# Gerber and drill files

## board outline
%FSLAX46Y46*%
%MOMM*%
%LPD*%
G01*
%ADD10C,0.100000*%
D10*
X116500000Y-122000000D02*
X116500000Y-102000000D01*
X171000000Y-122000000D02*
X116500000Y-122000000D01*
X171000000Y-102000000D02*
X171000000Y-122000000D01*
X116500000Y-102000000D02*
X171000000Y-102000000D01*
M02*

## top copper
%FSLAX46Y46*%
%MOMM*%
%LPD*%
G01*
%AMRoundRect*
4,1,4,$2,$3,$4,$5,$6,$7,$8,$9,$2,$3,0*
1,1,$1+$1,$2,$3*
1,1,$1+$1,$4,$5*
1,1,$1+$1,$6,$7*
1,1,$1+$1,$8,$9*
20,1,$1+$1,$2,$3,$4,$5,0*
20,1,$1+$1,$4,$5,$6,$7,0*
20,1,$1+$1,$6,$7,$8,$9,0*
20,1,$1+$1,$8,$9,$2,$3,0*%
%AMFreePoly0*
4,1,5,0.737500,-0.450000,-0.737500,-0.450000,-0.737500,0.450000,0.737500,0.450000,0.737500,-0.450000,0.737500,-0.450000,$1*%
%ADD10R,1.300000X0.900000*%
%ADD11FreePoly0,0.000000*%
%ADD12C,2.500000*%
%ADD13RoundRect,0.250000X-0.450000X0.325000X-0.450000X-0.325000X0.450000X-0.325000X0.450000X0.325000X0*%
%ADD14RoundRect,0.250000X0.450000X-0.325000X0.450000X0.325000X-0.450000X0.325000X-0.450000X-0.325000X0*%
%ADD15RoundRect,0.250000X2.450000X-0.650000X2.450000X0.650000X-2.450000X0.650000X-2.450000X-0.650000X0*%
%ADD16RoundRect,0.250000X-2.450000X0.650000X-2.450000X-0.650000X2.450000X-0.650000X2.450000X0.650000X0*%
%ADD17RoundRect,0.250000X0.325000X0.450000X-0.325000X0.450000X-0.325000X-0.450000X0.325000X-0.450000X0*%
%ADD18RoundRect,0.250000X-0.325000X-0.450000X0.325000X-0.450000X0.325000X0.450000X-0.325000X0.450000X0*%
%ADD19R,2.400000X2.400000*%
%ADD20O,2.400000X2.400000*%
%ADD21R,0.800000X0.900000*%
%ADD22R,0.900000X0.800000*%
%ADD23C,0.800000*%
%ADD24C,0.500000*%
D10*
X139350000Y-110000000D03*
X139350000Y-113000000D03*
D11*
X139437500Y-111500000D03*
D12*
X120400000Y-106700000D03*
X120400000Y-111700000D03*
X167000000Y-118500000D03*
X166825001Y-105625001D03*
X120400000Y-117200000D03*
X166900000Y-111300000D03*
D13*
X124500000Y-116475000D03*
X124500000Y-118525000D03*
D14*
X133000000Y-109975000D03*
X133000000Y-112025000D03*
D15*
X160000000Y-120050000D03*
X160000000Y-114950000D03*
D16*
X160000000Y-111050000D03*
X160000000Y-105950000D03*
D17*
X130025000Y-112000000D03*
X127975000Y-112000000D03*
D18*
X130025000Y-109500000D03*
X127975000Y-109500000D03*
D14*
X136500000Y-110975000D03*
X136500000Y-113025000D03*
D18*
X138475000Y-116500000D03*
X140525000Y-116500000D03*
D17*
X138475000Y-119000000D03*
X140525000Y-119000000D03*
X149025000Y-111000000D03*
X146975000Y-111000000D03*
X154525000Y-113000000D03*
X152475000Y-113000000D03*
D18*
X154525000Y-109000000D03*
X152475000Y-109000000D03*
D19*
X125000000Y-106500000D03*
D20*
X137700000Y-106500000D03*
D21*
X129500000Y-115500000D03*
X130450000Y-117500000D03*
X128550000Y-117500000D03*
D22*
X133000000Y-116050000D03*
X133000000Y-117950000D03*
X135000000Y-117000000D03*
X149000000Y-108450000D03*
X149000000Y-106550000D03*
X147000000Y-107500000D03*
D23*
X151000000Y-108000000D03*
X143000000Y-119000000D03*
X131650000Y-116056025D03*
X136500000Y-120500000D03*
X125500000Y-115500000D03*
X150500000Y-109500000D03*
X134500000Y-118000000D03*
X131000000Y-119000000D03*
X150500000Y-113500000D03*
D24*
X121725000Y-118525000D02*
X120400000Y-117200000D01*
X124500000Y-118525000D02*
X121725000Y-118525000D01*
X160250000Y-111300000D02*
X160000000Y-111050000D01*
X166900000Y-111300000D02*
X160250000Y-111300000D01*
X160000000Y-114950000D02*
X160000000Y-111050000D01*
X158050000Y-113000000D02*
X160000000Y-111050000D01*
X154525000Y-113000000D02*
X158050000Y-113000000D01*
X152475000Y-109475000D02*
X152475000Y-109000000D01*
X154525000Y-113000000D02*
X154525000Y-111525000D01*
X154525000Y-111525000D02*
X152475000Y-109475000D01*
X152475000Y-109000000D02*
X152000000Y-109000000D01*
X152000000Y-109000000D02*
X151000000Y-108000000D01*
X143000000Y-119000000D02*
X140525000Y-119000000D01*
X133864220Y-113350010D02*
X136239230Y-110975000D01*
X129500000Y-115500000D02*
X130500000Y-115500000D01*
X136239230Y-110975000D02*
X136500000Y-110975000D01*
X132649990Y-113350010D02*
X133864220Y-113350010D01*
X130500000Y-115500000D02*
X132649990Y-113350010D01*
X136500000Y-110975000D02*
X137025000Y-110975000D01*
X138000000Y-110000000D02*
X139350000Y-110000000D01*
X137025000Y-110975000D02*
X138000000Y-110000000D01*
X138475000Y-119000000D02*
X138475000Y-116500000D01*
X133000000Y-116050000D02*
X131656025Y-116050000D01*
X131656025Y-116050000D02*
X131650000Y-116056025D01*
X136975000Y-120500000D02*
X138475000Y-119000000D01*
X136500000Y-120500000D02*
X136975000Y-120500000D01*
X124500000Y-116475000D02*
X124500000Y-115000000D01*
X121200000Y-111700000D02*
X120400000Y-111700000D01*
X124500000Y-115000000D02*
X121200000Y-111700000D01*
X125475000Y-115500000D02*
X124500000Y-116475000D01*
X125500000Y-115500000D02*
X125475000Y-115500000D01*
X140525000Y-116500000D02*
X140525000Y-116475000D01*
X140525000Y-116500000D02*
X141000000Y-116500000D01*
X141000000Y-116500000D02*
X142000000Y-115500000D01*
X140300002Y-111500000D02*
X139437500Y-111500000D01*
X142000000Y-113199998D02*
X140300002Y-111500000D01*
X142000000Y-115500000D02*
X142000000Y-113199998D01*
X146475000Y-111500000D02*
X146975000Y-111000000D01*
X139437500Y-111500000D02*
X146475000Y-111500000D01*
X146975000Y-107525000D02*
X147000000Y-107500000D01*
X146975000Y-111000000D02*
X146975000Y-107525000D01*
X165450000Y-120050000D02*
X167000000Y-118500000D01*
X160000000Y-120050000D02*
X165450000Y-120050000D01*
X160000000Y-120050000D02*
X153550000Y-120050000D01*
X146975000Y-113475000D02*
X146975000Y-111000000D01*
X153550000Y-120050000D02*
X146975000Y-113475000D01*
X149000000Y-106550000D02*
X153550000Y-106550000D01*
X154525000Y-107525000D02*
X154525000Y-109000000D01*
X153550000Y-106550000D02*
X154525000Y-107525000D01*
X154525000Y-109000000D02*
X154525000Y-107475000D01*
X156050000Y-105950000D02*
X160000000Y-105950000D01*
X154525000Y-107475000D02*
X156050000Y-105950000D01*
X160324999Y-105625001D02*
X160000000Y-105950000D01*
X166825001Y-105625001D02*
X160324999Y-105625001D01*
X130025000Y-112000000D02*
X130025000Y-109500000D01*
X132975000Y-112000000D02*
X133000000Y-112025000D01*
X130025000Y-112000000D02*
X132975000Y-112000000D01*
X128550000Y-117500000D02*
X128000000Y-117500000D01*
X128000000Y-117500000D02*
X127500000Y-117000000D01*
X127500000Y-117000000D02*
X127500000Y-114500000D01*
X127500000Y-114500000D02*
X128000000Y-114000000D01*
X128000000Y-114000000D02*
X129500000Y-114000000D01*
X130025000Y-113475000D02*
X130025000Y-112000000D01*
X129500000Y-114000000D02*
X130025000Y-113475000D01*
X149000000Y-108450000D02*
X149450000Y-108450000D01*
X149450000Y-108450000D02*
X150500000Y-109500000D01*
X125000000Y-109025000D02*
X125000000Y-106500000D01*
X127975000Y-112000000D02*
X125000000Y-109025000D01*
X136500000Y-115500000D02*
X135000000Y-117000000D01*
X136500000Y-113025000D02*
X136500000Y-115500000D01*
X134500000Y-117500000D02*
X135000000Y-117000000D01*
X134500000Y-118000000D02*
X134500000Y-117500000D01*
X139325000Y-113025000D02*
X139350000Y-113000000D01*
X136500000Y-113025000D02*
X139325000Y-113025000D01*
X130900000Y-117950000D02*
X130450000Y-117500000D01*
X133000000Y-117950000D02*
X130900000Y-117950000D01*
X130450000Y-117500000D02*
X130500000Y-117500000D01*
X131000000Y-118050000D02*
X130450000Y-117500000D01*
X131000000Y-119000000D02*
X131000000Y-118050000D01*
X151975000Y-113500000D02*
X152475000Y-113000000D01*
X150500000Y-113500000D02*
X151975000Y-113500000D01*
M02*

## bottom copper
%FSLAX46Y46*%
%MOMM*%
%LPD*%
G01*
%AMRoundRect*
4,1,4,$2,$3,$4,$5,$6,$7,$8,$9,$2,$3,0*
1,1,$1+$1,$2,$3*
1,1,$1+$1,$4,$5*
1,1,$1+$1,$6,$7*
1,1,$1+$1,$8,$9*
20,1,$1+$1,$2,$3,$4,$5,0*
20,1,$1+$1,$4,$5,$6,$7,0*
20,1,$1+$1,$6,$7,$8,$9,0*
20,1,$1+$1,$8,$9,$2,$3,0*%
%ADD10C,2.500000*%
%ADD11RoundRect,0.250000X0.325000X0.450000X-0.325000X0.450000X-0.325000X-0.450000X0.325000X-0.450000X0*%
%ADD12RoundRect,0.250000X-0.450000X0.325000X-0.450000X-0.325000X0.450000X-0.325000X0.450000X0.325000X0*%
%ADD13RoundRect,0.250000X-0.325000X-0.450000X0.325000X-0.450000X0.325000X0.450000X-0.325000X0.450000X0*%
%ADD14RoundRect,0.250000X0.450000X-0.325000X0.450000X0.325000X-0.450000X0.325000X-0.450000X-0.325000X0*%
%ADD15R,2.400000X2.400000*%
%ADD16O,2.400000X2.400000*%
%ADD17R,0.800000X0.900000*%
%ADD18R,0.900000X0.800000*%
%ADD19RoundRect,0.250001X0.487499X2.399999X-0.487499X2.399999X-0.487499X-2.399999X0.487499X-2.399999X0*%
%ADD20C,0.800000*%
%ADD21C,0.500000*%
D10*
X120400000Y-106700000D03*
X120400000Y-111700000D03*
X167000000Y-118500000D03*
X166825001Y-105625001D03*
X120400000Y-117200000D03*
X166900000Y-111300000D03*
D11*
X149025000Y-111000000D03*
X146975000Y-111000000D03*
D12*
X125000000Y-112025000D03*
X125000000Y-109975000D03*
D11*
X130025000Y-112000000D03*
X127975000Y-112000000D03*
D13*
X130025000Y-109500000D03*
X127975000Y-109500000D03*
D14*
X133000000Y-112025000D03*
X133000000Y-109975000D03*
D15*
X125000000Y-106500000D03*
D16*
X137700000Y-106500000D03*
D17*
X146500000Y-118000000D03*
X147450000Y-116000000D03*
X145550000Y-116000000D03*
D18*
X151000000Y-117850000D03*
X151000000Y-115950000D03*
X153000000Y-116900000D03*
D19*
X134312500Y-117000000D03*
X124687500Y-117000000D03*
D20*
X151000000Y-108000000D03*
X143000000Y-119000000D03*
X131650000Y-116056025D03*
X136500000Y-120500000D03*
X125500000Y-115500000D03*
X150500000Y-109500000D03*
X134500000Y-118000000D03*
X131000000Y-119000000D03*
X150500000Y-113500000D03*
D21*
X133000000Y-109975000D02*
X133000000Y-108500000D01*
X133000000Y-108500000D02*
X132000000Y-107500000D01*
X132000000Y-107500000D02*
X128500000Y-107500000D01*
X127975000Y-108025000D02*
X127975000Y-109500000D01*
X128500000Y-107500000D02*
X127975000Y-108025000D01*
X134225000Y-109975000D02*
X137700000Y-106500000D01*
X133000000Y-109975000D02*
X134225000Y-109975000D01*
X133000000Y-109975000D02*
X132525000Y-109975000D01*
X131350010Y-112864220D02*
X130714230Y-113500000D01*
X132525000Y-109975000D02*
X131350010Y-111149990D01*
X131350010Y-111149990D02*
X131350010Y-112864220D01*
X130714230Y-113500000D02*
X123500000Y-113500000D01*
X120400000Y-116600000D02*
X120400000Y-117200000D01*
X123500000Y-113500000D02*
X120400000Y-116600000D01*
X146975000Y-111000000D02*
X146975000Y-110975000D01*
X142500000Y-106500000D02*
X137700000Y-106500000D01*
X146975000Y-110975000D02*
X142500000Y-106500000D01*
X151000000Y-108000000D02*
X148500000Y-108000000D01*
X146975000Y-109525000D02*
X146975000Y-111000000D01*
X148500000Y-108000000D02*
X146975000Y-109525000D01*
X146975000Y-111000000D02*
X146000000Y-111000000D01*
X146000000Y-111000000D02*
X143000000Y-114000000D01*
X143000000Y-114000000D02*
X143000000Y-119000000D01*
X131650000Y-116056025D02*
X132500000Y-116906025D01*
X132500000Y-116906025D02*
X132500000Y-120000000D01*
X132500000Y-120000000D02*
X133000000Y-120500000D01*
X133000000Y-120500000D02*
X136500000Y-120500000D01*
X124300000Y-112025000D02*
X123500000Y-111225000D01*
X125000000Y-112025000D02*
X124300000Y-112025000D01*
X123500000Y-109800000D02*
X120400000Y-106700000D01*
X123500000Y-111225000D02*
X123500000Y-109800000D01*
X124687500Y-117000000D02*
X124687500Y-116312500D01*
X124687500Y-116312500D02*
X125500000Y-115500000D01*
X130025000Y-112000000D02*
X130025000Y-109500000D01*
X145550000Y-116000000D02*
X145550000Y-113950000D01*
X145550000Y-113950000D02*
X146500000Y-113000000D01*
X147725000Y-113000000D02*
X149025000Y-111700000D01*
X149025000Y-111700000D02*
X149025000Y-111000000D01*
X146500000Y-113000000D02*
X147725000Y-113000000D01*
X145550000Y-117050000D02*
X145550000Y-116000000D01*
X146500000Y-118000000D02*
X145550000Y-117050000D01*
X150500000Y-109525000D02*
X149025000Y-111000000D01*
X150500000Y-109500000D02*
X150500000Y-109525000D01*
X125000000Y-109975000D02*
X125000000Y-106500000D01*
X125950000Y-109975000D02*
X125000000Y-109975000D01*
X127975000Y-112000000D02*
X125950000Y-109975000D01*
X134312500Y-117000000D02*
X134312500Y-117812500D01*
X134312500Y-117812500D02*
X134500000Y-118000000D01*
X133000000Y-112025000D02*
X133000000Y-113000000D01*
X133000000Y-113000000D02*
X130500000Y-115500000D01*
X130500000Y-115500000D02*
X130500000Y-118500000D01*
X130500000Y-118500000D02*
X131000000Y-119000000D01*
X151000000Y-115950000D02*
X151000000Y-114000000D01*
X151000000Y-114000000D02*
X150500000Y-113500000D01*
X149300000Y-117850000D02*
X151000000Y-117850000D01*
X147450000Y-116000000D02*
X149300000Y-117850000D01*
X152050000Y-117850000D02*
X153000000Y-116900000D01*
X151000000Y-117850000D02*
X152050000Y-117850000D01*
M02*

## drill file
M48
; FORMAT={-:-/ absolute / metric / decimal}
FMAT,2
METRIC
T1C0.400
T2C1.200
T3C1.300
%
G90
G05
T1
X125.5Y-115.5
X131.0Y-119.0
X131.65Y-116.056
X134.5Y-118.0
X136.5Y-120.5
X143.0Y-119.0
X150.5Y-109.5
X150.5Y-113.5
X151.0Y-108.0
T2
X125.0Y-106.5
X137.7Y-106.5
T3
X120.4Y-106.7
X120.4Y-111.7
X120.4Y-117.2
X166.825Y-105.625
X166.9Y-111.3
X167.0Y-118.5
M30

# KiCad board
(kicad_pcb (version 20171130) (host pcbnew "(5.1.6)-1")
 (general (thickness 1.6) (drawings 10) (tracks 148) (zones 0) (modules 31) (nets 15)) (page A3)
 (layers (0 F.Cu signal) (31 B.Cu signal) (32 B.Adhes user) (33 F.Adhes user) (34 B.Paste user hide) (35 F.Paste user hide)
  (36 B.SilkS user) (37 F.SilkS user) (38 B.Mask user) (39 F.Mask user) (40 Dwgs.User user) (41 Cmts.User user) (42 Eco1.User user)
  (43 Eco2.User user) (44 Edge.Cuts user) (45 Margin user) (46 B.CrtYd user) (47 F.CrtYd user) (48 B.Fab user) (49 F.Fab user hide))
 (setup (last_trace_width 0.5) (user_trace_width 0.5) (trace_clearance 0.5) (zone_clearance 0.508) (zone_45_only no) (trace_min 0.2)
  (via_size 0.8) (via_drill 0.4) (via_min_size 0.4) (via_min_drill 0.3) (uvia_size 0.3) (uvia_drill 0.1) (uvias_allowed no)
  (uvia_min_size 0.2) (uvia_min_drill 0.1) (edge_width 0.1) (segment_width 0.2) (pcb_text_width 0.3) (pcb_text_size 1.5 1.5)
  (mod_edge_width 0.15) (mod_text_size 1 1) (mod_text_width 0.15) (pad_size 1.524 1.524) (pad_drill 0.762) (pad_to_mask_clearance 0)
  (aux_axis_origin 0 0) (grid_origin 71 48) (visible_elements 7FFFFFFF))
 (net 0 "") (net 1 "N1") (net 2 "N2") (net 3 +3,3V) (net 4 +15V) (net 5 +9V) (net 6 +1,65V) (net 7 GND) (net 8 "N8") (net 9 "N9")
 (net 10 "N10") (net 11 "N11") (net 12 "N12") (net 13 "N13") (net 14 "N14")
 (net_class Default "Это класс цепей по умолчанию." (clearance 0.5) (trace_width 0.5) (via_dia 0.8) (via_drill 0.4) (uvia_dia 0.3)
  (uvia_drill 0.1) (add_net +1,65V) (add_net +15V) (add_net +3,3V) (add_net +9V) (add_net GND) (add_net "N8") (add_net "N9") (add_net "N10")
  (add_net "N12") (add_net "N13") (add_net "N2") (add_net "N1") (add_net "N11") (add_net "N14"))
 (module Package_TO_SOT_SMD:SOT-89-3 (layer F.Cu) (at 141 111.5)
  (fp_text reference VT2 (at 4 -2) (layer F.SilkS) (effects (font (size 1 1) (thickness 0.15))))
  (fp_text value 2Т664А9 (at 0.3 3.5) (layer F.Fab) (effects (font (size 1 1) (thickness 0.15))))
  (pad 1 smd rect (at -1.65 -1.5) (size 1.3 0.9) (layers F.Cu F.Paste F.Mask) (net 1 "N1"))
  (pad 3 smd rect (at -1.65 1.5) (size 1.3 0.9) (layers F.Cu F.Paste F.Mask) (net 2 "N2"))
  (pad 2 smd custom (at -1.5625 0) (size 1.475 0.9) (layers F.Cu F.Paste F.Mask) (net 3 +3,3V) (zone_connect 2)
   (options (clearance outline) (anchor rect)) (primitives)))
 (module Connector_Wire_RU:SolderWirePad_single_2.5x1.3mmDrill (layer F.Cu) (at 120.4 106.7)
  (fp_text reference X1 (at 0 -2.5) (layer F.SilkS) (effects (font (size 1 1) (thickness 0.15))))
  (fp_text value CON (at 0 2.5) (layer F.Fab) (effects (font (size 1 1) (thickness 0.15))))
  (pad 1 thru_hole circle (at 0 0) (size 2.5 2.5) (drill 1.3) (layers *.Cu *.Mask) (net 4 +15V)))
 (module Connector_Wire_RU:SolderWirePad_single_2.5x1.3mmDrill (layer F.Cu) (at 120.4 111.7)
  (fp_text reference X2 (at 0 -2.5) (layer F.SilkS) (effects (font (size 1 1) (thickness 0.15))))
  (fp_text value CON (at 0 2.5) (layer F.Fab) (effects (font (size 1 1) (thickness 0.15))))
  (pad 1 thru_hole circle (at 0 0) (size 2.5 2.5) (drill 1.3) (layers *.Cu *.Mask) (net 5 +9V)))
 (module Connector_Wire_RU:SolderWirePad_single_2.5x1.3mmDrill (layer F.Cu) (at 167 118.5)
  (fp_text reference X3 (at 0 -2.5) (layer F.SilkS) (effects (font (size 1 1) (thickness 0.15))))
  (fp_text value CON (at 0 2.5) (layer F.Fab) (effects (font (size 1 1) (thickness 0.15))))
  (pad 1 thru_hole circle (at 0 0) (size 2.5 2.5) (drill 1.3) (layers *.Cu *.Mask) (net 3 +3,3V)))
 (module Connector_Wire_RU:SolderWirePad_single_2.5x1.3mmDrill (layer F.Cu) (at 166.825001 105.625001)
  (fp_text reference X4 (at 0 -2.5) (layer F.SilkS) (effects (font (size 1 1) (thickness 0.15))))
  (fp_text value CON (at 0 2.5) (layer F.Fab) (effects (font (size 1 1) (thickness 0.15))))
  (pad 1 thru_hole circle (at 0 0) (size 2.5 2.5) (drill 1.3) (layers *.Cu *.Mask) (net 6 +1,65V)))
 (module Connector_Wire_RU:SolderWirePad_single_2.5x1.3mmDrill (layer F.Cu) (at 120.4 117.2)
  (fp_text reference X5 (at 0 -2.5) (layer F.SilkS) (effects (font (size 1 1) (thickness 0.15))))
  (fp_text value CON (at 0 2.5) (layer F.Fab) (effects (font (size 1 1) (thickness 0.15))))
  (pad 1 thru_hole circle (at 0 0) (size 2.5 2.5) (drill 1.3) (layers *.Cu *.Mask) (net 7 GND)))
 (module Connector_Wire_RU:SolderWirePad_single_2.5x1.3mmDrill (layer F.Cu) (at 166.9 111.3)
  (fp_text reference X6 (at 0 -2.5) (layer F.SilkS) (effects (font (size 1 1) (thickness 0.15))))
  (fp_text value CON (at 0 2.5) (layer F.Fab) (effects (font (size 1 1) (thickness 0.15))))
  (pad 1 thru_hole circle (at 0 0) (size 2.5 2.5) (drill 1.3) (layers *.Cu *.Mask) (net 7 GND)))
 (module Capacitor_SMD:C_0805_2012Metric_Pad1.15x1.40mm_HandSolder (layer F.Cu) (at 124.5 117.5 270)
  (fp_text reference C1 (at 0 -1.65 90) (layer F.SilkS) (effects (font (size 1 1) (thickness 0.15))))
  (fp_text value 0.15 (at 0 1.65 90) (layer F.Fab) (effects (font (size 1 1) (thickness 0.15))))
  (pad 1 smd roundrect (at -1.025 0 270) (size 1.15 1.4) (layers F.Cu F.Paste F.Mask) (roundrect_rratio 0.217391) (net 5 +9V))
  (pad 2 smd roundrect (at 1.025 0 270) (size 1.15 1.4) (layers F.Cu F.Paste F.Mask) (roundrect_rratio 0.217391) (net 7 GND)))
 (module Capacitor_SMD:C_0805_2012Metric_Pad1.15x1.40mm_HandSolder (layer F.Cu) (at 133 111 90)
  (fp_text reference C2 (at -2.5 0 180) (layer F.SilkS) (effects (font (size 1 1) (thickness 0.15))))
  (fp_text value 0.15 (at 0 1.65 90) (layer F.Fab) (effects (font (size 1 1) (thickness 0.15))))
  (pad 2 smd roundrect (at 1.025 0 90) (size 1.15 1.4) (layers F.Cu F.Paste F.Mask) (roundrect_rratio 0.217391) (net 7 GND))
  (pad 1 smd roundrect (at -1.025 0 90) (size 1.15 1.4) (layers F.Cu F.Paste F.Mask) (roundrect_rratio 0.217391) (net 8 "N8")))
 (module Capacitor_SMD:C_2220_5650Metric (layer F.Cu) (at 160 117.5 90)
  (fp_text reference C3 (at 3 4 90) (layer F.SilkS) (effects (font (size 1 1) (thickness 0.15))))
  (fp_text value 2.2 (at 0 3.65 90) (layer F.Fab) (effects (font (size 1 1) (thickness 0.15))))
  (pad 1 smd roundrect (at -2.55 0 90) (size 1.8 5.4) (layers F.Cu F.Paste F.Mask) (roundrect_rratio 0.138889) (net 3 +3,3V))
  (pad 2 smd roundrect (at 2.55 0 90) (size 1.8 5.4) (layers F.Cu F.Paste F.Mask) (roundrect_rratio 0.138889) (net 7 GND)))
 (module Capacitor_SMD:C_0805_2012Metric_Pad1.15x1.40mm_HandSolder (layer B.Cu) (at 148 111 180)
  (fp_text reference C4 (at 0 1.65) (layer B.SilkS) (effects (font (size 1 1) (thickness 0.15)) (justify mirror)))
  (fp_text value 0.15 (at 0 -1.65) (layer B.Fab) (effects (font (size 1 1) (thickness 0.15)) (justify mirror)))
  (pad 1 smd roundrect (at -1.025 0 180) (size 1.15 1.4) (layers B.Cu B.Paste B.Mask) (roundrect_rratio 0.217391) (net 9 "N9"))
  (pad 2 smd roundrect (at 1.025 0 180) (size 1.15 1.4) (layers B.Cu B.Paste B.Mask) (roundrect_rratio 0.217391) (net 7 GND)))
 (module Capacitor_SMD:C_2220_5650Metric (layer F.Cu) (at 160 108.5 270)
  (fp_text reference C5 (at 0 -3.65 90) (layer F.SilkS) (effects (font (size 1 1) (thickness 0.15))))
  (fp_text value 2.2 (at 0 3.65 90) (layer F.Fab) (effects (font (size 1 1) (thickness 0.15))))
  (pad 2 smd roundrect (at 2.55 0 270) (size 1.8 5.4) (layers F.Cu F.Paste F.Mask) (roundrect_rratio 0.138889) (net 7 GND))
  (pad 1 smd roundrect (at -2.55 0 270) (size 1.8 5.4) (layers F.Cu F.Paste F.Mask) (roundrect_rratio 0.138889) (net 6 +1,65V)))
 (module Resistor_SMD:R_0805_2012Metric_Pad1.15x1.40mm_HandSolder (layer B.Cu) (at 125 111 270)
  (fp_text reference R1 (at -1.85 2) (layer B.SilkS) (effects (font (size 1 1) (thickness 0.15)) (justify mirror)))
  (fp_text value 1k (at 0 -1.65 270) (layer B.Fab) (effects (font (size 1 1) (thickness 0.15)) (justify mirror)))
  (pad 2 smd roundrect (at 1.025 0 270) (size 1.15 1.4) (layers B.Cu B.Paste B.Mask) (roundrect_rratio 0.217391) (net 4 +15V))
  (pad 1 smd roundrect (at -1.025 0 270) (size 1.15 1.4) (layers B.Cu B.Paste B.Mask) (roundrect_rratio 0.217391) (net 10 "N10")))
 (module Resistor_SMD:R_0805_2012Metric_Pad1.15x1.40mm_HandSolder (layer F.Cu) (at 129 112 180)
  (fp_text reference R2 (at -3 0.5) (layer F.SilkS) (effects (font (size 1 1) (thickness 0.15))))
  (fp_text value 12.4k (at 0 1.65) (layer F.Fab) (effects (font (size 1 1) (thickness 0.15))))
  (pad 1 smd roundrect (at -1.025 0 180) (size 1.15 1.4) (layers F.Cu F.Paste F.Mask) (roundrect_rratio 0.217391) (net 8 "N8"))
  (pad 2 smd roundrect (at 1.025 0 180) (size 1.15 1.4) (layers F.Cu F.Paste F.Mask) (roundrect_rratio 0.217391) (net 10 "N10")))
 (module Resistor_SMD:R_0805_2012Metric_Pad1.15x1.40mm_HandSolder (layer F.Cu) (at 129 109.5)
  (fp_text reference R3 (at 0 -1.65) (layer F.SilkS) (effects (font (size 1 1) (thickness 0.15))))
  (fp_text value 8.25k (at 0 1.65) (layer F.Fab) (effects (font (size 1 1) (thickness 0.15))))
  (pad 2 smd roundrect (at 1.025 0) (size 1.15 1.4) (layers F.Cu F.Paste F.Mask) (roundrect_rratio 0.217391) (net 8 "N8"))
  (pad 1 smd roundrect (at -1.025 0) (size 1.15 1.4) (layers F.Cu F.Paste F.Mask) (roundrect_rratio 0.217391) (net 7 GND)))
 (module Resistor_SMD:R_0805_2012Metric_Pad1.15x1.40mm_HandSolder (layer B.Cu) (at 129 112 180)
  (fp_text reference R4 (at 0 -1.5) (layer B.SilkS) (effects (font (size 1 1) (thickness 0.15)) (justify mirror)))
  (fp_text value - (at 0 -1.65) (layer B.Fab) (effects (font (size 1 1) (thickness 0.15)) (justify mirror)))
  (pad 1 smd roundrect (at -1.025 0 180) (size 1.15 1.4) (layers B.Cu B.Paste B.Mask) (roundrect_rratio 0.217391) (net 8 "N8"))
  (pad 2 smd roundrect (at 1.025 0 180) (size 1.15 1.4) (layers B.Cu B.Paste B.Mask) (roundrect_rratio 0.217391) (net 10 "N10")))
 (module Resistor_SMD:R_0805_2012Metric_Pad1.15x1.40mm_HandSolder (layer B.Cu) (at 129 109.5)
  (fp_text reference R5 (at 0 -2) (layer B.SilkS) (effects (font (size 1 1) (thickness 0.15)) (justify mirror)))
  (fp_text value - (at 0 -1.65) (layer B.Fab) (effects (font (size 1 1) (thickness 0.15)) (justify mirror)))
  (pad 2 smd roundrect (at 1.025 0) (size 1.15 1.4) (layers B.Cu B.Paste B.Mask) (roundrect_rratio 0.217391) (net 8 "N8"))
  (pad 1 smd roundrect (at -1.025 0) (size 1.15 1.4) (layers B.Cu B.Paste B.Mask) (roundrect_rratio 0.217391) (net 7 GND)))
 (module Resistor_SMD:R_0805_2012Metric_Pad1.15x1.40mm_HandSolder (layer F.Cu) (at 136.5 112 90)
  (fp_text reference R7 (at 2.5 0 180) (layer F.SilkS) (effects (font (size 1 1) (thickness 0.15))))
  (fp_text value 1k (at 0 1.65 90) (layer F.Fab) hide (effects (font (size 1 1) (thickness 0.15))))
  (pad 2 smd roundrect (at 1.025 0 90) (size 1.15 1.4) (layers F.Cu F.Paste F.Mask) (roundrect_rratio 0.217391) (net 1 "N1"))
  (pad 1 smd roundrect (at -1.025 0 90) (size 1.15 1.4) (layers F.Cu F.Paste F.Mask) (roundrect_rratio 0.217391) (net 2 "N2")))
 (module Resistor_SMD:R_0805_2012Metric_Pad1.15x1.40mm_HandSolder (layer B.Cu) (at 133 111 90)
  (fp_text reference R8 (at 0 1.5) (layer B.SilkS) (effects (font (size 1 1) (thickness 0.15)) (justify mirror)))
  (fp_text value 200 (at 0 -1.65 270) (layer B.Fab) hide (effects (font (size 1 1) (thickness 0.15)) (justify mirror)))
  (pad 1 smd roundrect (at -1.025 0 90) (size 1.15 1.4) (layers B.Cu B.Paste B.Mask) (roundrect_rratio 0.217391) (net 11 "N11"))
  (pad 2 smd roundrect (at 1.025 0 90) (size 1.15 1.4) (layers B.Cu B.Paste B.Mask) (roundrect_rratio 0.217391) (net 7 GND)))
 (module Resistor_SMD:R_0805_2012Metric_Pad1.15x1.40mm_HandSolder (layer F.Cu) (at 139.5 116.5)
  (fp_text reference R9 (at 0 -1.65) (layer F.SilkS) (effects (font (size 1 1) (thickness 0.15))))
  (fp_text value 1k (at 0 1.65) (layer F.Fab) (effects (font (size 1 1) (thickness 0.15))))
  (pad 1 smd roundrect (at -1.025 0) (size 1.15 1.4) (layers F.Cu F.Paste F.Mask) (roundrect_rratio 0.217391) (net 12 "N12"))
  (pad 2 smd roundrect (at 1.025 0) (size 1.15 1.4) (layers F.Cu F.Paste F.Mask) (roundrect_rratio 0.217391) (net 3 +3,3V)))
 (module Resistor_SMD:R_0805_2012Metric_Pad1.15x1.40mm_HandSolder (layer F.Cu) (at 139.5 119 180)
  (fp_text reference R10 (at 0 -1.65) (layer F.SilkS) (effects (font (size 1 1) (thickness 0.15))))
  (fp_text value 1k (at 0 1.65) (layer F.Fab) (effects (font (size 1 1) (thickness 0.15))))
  (pad 2 smd roundrect (at 1.025 0 180) (size 1.15 1.4) (layers F.Cu F.Paste F.Mask) (roundrect_rratio 0.217391) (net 12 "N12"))
  (pad 1 smd roundrect (at -1.025 0 180) (size 1.15 1.4) (layers F.Cu F.Paste F.Mask) (roundrect_rratio 0.217391) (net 7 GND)))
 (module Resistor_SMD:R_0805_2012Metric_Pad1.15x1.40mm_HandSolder (layer F.Cu) (at 148 111 180)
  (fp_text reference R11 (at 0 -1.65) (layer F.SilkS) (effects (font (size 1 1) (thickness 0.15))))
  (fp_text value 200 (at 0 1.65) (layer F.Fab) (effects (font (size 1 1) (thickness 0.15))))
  (pad 1 smd roundrect (at -1.025 0 180) (size 1.15 1.4) (layers F.Cu F.Paste F.Mask) (roundrect_rratio 0.217391) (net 9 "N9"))
  (pad 2 smd roundrect (at 1.025 0 180) (size 1.15 1.4) (layers F.Cu F.Paste F.Mask) (roundrect_rratio 0.217391) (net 3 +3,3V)))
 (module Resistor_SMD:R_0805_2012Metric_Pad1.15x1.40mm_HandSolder (layer F.Cu) (at 153.5 113 180)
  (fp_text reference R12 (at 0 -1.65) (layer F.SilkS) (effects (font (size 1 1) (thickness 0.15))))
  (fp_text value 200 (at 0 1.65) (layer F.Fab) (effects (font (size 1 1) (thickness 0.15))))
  (pad 1 smd roundrect (at -1.025 0 180) (size 1.15 1.4) (layers F.Cu F.Paste F.Mask) (roundrect_rratio 0.217391) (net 7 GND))
  (pad 2 smd roundrect (at 1.025 0 180) (size 1.15 1.4) (layers F.Cu F.Paste F.Mask) (roundrect_rratio 0.217391) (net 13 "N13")))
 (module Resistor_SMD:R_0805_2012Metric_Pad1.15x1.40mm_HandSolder (layer F.Cu) (at 153.5 109)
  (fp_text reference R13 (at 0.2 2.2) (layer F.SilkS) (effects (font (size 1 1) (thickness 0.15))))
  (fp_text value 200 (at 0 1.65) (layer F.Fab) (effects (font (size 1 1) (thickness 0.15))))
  (pad 2 smd roundrect (at 1.025 0) (size 1.15 1.4) (layers F.Cu F.Paste F.Mask) (roundrect_rratio 0.217391) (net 6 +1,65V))
  (pad 1 smd roundrect (at -1.025 0) (size 1.15 1.4) (layers F.Cu F.Paste F.Mask) (roundrect_rratio 0.217391) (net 7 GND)))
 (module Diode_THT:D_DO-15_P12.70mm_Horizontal (layer F.Cu) (at 125 106.5)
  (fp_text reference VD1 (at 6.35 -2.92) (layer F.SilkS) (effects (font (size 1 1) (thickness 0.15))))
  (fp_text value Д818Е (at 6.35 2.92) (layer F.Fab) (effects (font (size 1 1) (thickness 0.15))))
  (pad 1 thru_hole rect (at 0 0) (size 2.4 2.4) (drill 1.2) (layers *.Cu *.Mask) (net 10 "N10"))
  (pad 2 thru_hole oval (at 12.7 0) (size 2.4 2.4) (drill 1.2) (layers *.Cu *.Mask) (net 7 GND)))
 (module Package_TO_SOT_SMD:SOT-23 (layer F.Cu) (at 129.5 116.5 90)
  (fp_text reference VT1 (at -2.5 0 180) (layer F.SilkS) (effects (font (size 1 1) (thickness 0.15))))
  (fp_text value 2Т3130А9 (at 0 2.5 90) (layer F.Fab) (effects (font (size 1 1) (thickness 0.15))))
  (pad 3 smd rect (at 1 0 90) (size 0.9 0.8) (layers F.Cu F.Paste F.Mask) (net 1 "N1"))
  (pad 2 smd rect (at -1 0.95 90) (size 0.9 0.8) (layers F.Cu F.Paste F.Mask) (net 11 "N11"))
  (pad 1 smd rect (at -1 -0.95 90) (size 0.9 0.8) (layers F.Cu F.Paste F.Mask) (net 8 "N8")))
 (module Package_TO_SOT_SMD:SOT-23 (layer F.Cu) (at 134 117)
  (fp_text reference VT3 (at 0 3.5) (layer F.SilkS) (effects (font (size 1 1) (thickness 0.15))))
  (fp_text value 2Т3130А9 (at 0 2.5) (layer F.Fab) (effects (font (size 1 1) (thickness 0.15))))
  (pad 1 smd rect (at -1 -0.95) (size 0.9 0.8) (layers F.Cu F.Paste F.Mask) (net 12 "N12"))
  (pad 2 smd rect (at -1 0.95) (size 0.9 0.8) (layers F.Cu F.Paste F.Mask) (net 11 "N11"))
  (pad 3 smd rect (at 1 0) (size 0.9 0.8) (layers F.Cu F.Paste F.Mask) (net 2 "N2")))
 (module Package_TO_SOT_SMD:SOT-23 (layer B.Cu) (at 146.5 117 270)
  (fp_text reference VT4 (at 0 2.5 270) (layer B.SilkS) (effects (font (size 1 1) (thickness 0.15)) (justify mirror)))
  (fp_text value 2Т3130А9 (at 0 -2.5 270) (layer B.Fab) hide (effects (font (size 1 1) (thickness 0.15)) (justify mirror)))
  (pad 3 smd rect (at 1 0 270) (size 0.9 0.8) (layers B.Cu B.Paste B.Mask) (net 9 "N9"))
  (pad 2 smd rect (at -1 -0.95 270) (size 0.9 0.8) (layers B.Cu B.Paste B.Mask) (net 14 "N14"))
  (pad 1 smd rect (at -1 0.95 270) (size 0.9 0.8) (layers B.Cu B.Paste B.Mask) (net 9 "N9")))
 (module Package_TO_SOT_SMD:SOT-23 (layer B.Cu) (at 152 116.9)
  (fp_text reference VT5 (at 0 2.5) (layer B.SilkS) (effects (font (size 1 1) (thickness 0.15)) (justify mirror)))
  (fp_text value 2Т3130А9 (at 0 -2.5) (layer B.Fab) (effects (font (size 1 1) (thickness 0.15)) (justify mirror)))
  (pad 1 smd rect (at -1 0.95) (size 0.9 0.8) (layers B.Cu B.Paste B.Mask) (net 14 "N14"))
  (pad 2 smd rect (at -1 -0.95) (size 0.9 0.8) (layers B.Cu B.Paste B.Mask) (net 13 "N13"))
  (pad 3 smd rect (at 1 0) (size 0.9 0.8) (layers B.Cu B.Paste B.Mask) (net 14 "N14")))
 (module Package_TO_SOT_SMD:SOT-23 (layer F.Cu) (at 148 107.5 180)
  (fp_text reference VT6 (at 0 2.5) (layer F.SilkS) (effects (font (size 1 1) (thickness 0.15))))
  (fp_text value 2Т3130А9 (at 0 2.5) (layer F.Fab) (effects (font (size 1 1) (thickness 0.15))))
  (pad 1 smd rect (at -1 -0.95 180) (size 0.9 0.8) (layers F.Cu F.Paste F.Mask) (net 9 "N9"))
  (pad 2 smd rect (at -1 0.95 180) (size 0.9 0.8) (layers F.Cu F.Paste F.Mask) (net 6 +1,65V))
  (pad 3 smd rect (at 1 0 180) (size 0.9 0.8) (layers F.Cu F.Paste F.Mask) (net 3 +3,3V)))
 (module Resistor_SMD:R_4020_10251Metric (layer B.Cu) (at 129.5 117 180)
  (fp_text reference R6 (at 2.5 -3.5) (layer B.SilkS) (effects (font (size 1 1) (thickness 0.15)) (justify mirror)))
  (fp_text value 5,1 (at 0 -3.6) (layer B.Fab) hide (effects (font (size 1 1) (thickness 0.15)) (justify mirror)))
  (pad 1 smd roundrect (at -4.8125 0 180) (size 1.475 5.3) (layers B.Cu B.Paste B.Mask) (roundrect_rratio 0.169492) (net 2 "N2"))
  (pad 2 smd roundrect (at 4.8125 0 180) (size 1.475 5.3) (layers B.Cu B.Paste B.Mask) (roundrect_rratio 0.169492) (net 5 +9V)))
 (gr_line (start 116.5 122) (end 116.5 102) (layer Edge.Cuts) (width 0.1))
 (gr_line (start 171 122) (end 116.5 122) (layer Edge.Cuts) (width 0.1))
 (gr_line (start 171 102) (end 171 122) (layer Edge.Cuts) (width 0.1))
 (gr_line (start 116.5 102) (end 171 102) (layer Edge.Cuts) (width 0.1))
 (segment (start 121.725 118.525) (end 120.4 117.2) (width 0.5) (layer F.Cu) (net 7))
 (segment (start 124.5 118.525) (end 121.725 118.525) (width 0.5) (layer F.Cu) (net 7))
 (segment (start 133 109.975) (end 133 108.5) (width 0.5) (layer B.Cu) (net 7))
 (segment (start 133 108.5) (end 132 107.5) (width 0.5) (layer B.Cu) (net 7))
 (segment (start 132 107.5) (end 128.5 107.5) (width 0.5) (layer B.Cu) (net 7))
 (segment (start 127.975 108.025) (end 127.975 109.5) (width 0.5) (layer B.Cu) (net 7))
 (segment (start 128.5 107.5) (end 127.975 108.025) (width 0.5) (layer B.Cu) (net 7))
 (segment (start 134.225 109.975) (end 137.7 106.5) (width 0.5) (layer B.Cu) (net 7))
 (segment (start 133 109.975) (end 134.225 109.975) (width 0.5) (layer B.Cu) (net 7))
 (segment (start 133 109.975) (end 132.525 109.975) (width 0.5) (layer B.Cu) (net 7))
 (segment (start 131.35001 112.86422) (end 130.71423 113.5) (width 0.5) (layer B.Cu) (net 7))
 (segment (start 132.525 109.975) (end 131.35001 111.14999) (width 0.5) (layer B.Cu) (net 7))
 (segment (start 131.35001 111.14999) (end 131.35001 112.86422) (width 0.5) (layer B.Cu) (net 7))
 (segment (start 130.71423 113.5) (end 123.5 113.5) (width 0.5) (layer B.Cu) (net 7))
 (segment (start 120.4 116.6) (end 120.4 117.2) (width 0.5) (layer B.Cu) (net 7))
 (segment (start 123.5 113.5) (end 120.4 116.6) (width 0.5) (layer B.Cu) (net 7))
 (segment (start 160.25 111.3) (end 160 111.05) (width 0.5) (layer F.Cu) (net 7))
 (segment (start 166.9 111.3) (end 160.25 111.3) (width 0.5) (layer F.Cu) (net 7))
 (segment (start 160 114.95) (end 160 111.05) (width 0.5) (layer F.Cu) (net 7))
 (segment (start 158.05 113) (end 160 111.05) (width 0.5) (layer F.Cu) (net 7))
 (segment (start 154.525 113) (end 158.05 113) (width 0.5) (layer F.Cu) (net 7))
 (segment (start 146.975 111) (end 146.975 110.975) (width 0.5) (layer B.Cu) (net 7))
 (segment (start 142.5 106.5) (end 137.7 106.5) (width 0.5) (layer B.Cu) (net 7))
 (segment (start 146.975 110.975) (end 142.5 106.5) (width 0.5) (layer B.Cu) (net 7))
 (segment (start 152.475 109.475) (end 152.475 109) (width 0.5) (layer F.Cu) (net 7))
 (segment (start 154.525 113) (end 154.525 111.525) (width 0.5) (layer F.Cu) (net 7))
 (segment (start 154.525 111.525) (end 152.475 109.475) (width 0.5) (layer F.Cu) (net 7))
 (via (at 151 108) (size 0.8) (drill 0.4) (layers F.Cu B.Cu) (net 7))
 (segment (start 152.475 109) (end 152 109) (width 0.5) (layer F.Cu) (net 7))
 (segment (start 152 109) (end 151 108) (width 0.5) (layer F.Cu) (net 7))
 (segment (start 151 108) (end 148.5 108) (width 0.5) (layer B.Cu) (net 7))
 (segment (start 146.975 109.525) (end 146.975 111) (width 0.5) (layer B.Cu) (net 7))
 (segment (start 148.5 108) (end 146.975 109.525) (width 0.5) (layer B.Cu) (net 7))
 (segment (start 146.975 111) (end 146 111) (width 0.5) (layer B.Cu) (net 7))
 (via (at 143 119) (size 0.8) (drill 0.4) (layers F.Cu B.Cu) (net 7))
 (segment (start 146 111) (end 143 114) (width 0.5) (layer B.Cu) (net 7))
 (segment (start 143 114) (end 143 119) (width 0.5) (layer B.Cu) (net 7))
 (segment (start 143 119) (end 140.525 119) (width 0.5) (layer F.Cu) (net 7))
 (segment (start 133.86422 113.35001) (end 136.23923 110.975) (width 0.5) (layer F.Cu) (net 1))
 (segment (start 129.5 115.5) (end 130.5 115.5) (width 0.5) (layer F.Cu) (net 1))
 (segment (start 136.23923 110.975) (end 136.5 110.975) (width 0.5) (layer F.Cu) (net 1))
 (segment (start 132.64999 113.35001) (end 133.86422 113.35001) (width 0.5) (layer F.Cu) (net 1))
 (segment (start 130.5 115.5) (end 132.64999 113.35001) (width 0.5) (layer F.Cu) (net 1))
 (segment (start 136.5 110.975) (end 137.025 110.975) (width 0.5) (layer F.Cu) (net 1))
 (segment (start 138 110) (end 139.35 110) (width 0.5) (layer F.Cu) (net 1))
 (segment (start 137.025 110.975) (end 138 110) (width 0.5) (layer F.Cu) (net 1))
 (segment (start 138.475 119) (end 138.475 116.5) (width 0.5) (layer F.Cu) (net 12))
 (via (at 131.65 116.056025) (size 0.8) (drill 0.4) (layers F.Cu B.Cu) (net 12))
 (segment (start 133 116.05) (end 131.656025 116.05) (width 0.5) (layer F.Cu) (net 12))
 (segment (start 131.656025 116.05) (end 131.65 116.056025) (width 0.5) (layer F.Cu) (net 12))
 (segment (start 131.65 116.056025) (end 132.5 116.906025) (width 0.5) (layer B.Cu) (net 12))
 (segment (start 132.5 116.906025) (end 132.5 120) (width 0.5) (layer B.Cu) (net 12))
 (via (at 136.5 120.5) (size 0.8) (drill 0.4) (layers F.Cu B.Cu) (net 12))
 (segment (start 132.5 120) (end 133 120.5) (width 0.5) (layer B.Cu) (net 12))
 (segment (start 133 120.5) (end 136.5 120.5) (width 0.5) (layer B.Cu) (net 12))
 (segment (start 136.975 120.5) (end 138.475 119) (width 0.5) (layer F.Cu) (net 12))
 (segment (start 136.5 120.5) (end 136.975 120.5) (width 0.5) (layer F.Cu) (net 12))
 (segment (start 124.3 112.025) (end 123.5 111.225) (width 0.5) (layer B.Cu) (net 4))
 (segment (start 125 112.025) (end 124.3 112.025) (width 0.5) (layer B.Cu) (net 4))
 (segment (start 123.5 109.8) (end 120.4 106.7) (width 0.5) (layer B.Cu) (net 4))
 (segment (start 123.5 111.225) (end 123.5 109.8) (width 0.5) (layer B.Cu) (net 4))
 (segment (start 124.5 116.475) (end 124.5 115) (width 0.5) (layer F.Cu) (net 5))
 (segment (start 121.2 111.7) (end 120.4 111.7) (width 0.5) (layer F.Cu) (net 5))
 (segment (start 124.5 115) (end 121.2 111.7) (width 0.5) (layer F.Cu) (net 5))
 (via (at 125.5 115.5) (size 0.8) (drill 0.4) (layers F.Cu B.Cu) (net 5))
 (segment (start 124.6875 117) (end 124.6875 116.3125) (width 0.5) (layer B.Cu) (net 5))
 (segment (start 124.6875 116.3125) (end 125.5 115.5) (width 0.5) (layer B.Cu) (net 5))
 (segment (start 125.475 115.5) (end 124.5 116.475) (width 0.5) (layer F.Cu) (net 5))
 (segment (start 125.5 115.5) (end 125.475 115.5) (width 0.5) (layer F.Cu) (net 5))
 (segment (start 140.525 116.5) (end 140.525 116.475) (width 0.5) (layer F.Cu) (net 3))
 (segment (start 140.525 116.5) (end 141 116.5) (width 0.5) (layer F.Cu) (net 3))
 (segment (start 141 116.5) (end 142 115.5) (width 0.5) (layer F.Cu) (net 3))
 (segment (start 140.300002 111.5) (end 139.4375 111.5) (width 0.5) (layer F.Cu) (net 3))
 (segment (start 142 113.199998) (end 140.300002 111.5) (width 0.5) (layer F.Cu) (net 3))
 (segment (start 142 115.5) (end 142 113.199998) (width 0.5) (layer F.Cu) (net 3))
 (segment (start 146.475 111.5) (end 146.975 111) (width 0.5) (layer F.Cu) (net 3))
 (segment (start 139.4375 111.5) (end 146.475 111.5) (width 0.5) (layer F.Cu) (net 3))
 (segment (start 146.975 107.525) (end 147 107.5) (width 0.5) (layer F.Cu) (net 3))
 (segment (start 146.975 111) (end 146.975 107.525) (width 0.5) (layer F.Cu) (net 3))
 (segment (start 165.45 120.05) (end 167 118.5) (width 0.5) (layer F.Cu) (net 3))
 (segment (start 160 120.05) (end 165.45 120.05) (width 0.5) (layer F.Cu) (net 3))
 (segment (start 160 120.05) (end 153.55 120.05) (width 0.5) (layer F.Cu) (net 3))
 (segment (start 146.975 113.475) (end 146.975 111) (width 0.5) (layer F.Cu) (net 3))
 (segment (start 153.55 120.05) (end 146.975 113.475) (width 0.5) (layer F.Cu) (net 3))
 (segment (start 149 106.55) (end 153.55 106.55) (width 0.5) (layer F.Cu) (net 6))
 (segment (start 154.525 107.525) (end 154.525 109) (width 0.5) (layer F.Cu) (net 6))
 (segment (start 153.55 106.55) (end 154.525 107.525) (width 0.5) (layer F.Cu) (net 6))
 (segment (start 154.525 109) (end 154.525 107.475) (width 0.5) (layer F.Cu) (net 6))
 (segment (start 156.05 105.95) (end 160 105.95) (width 0.5) (layer F.Cu) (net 6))
 (segment (start 154.525 107.475) (end 156.05 105.95) (width 0.5) (layer F.Cu) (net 6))
 (segment (start 160.324999 105.625001) (end 160 105.95) (width 0.5) (layer F.Cu) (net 6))
 (segment (start 166.825001 105.625001) (end 160.324999 105.625001) (width 0.5) (layer F.Cu) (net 6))
 (segment (start 130.025 112) (end 130.025 109.5) (width 0.5) (layer F.Cu) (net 8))
 (segment (start 132.975 112) (end 133 112.025) (width 0.5) (layer F.Cu) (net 8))
 (segment (start 130.025 112) (end 132.975 112) (width 0.5) (layer F.Cu) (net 8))
 (segment (start 128.55 117.5) (end 128 117.5) (width 0.5) (layer F.Cu) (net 8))
 (segment (start 128 117.5) (end 127.5 117) (width 0.5) (layer F.Cu) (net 8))
 (segment (start 127.5 117) (end 127.5 114.5) (width 0.5) (layer F.Cu) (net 8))
 (segment (start 127.5 114.5) (end 128 114) (width 0.5) (layer F.Cu) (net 8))
 (segment (start 128 114) (end 129.5 114) (width 0.5) (layer F.Cu) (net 8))
 (segment (start 130.025 113.475) (end 130.025 112) (width 0.5) (layer F.Cu) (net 8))
 (segment (start 129.5 114) (end 130.025 113.475) (width 0.5) (layer F.Cu) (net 8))
 (segment (start 130.025 112) (end 130.025 109.5) (width 0.5) (layer B.Cu) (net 8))
 (segment (start 145.55 116) (end 145.55 113.95) (width 0.5) (layer B.Cu) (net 9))
 (segment (start 145.55 113.95) (end 146.5 113) (width 0.5) (layer B.Cu) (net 9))
 (segment (start 147.725 113) (end 149.025 111.7) (width 0.5) (layer B.Cu) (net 9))
 (segment (start 149.025 111.7) (end 149.025 111) (width 0.5) (layer B.Cu) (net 9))
 (segment (start 146.5 113) (end 147.725 113) (width 0.5) (layer B.Cu) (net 9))
 (segment (start 145.55 117.05) (end 145.55 116) (width 0.5) (layer B.Cu) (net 9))
 (segment (start 146.5 118) (end 145.55 117.05) (width 0.5) (layer B.Cu) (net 9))
 (via (at 150.5 109.5) (size 0.8) (drill 0.4) (layers F.Cu B.Cu) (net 9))
 (segment (start 149 108.45) (end 149.45 108.45) (width 0.5) (layer F.Cu) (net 9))
 (segment (start 149.45 108.45) (end 150.5 109.5) (width 0.5) (layer F.Cu) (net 9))
 (segment (start 150.5 109.525) (end 149.025 111) (width 0.5) (layer B.Cu) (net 9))
 (segment (start 150.5 109.5) (end 150.5 109.525) (width 0.5) (layer B.Cu) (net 9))
 (segment (start 125 109.975) (end 125 106.5) (width 0.5) (layer B.Cu) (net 10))
 (segment (start 125 109.025) (end 125 106.5) (width 0.5) (layer F.Cu) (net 10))
 (segment (start 127.975 112) (end 125 109.025) (width 0.5) (layer F.Cu) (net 10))
 (segment (start 125.95 109.975) (end 125 109.975) (width 0.5) (layer B.Cu) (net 10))
 (segment (start 127.975 112) (end 125.95 109.975) (width 0.5) (layer B.Cu) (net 10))
 (segment (start 136.5 115.5) (end 135 117) (width 0.5) (layer F.Cu) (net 2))
 (segment (start 136.5 113.025) (end 136.5 115.5) (width 0.5) (layer F.Cu) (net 2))
 (via (at 134.5 118) (size 0.8) (drill 0.4) (layers F.Cu B.Cu) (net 2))
 (segment (start 134.3125 117) (end 134.3125 117.8125) (width 0.5) (layer B.Cu) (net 2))
 (segment (start 134.3125 117.8125) (end 134.5 118) (width 0.5) (layer B.Cu) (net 2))
 (segment (start 134.5 117.5) (end 135 117) (width 0.5) (layer F.Cu) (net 2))
 (segment (start 134.5 118) (end 134.5 117.5) (width 0.5) (layer F.Cu) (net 2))
 (segment (start 139.325 113.025) (end 139.35 113) (width 0.5) (layer F.Cu) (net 2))
 (segment (start 136.5 113.025) (end 139.325 113.025) (width 0.5) (layer F.Cu) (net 2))
 (segment (start 130.9 117.95) (end 130.45 117.5) (width 0.5) (layer F.Cu) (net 11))
 (segment (start 133 117.95) (end 130.9 117.95) (width 0.5) (layer F.Cu) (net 11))
 (segment (start 130.45 117.5) (end 130.5 117.5) (width 0.5) (layer F.Cu) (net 11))
 (segment (start 133 112.025) (end 133 113) (width 0.5) (layer B.Cu) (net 11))
 (segment (start 133 113) (end 130.5 115.5) (width 0.5) (layer B.Cu) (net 11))
 (segment (start 130.5 115.5) (end 130.5 118.5) (width 0.5) (layer B.Cu) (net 11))
 (via (at 131 119) (size 0.8) (drill 0.4) (layers F.Cu B.Cu) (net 11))
 (segment (start 130.5 118.5) (end 131 119) (width 0.5) (layer B.Cu) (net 11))
 (segment (start 131 118.05) (end 130.45 117.5) (width 0.5) (layer F.Cu) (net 11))
 (segment (start 131 119) (end 131 118.05) (width 0.5) (layer F.Cu) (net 11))
 (via (at 150.5 113.5) (size 0.8) (drill 0.4) (layers F.Cu B.Cu) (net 13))
 (segment (start 151 115.95) (end 151 114) (width 0.5) (layer B.Cu) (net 13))
 (segment (start 151 114) (end 150.5 113.5) (width 0.5) (layer B.Cu) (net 13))
 (segment (start 151.975 113.5) (end 152.475 113) (width 0.5) (layer F.Cu) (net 13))
 (segment (start 150.5 113.5) (end 151.975 113.5) (width 0.5) (layer F.Cu) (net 13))
 (segment (start 149.3 117.85) (end 151 117.85) (width 0.5) (layer B.Cu) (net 14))
 (segment (start 147.45 116) (end 149.3 117.85) (width 0.5) (layer B.Cu) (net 14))
 (segment (start 152.05 117.85) (end 153 116.9) (width 0.5) (layer B.Cu) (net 14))
 (segment (start 151 117.85) (end 152.05 117.85) (width 0.5) (layer B.Cu) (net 14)))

